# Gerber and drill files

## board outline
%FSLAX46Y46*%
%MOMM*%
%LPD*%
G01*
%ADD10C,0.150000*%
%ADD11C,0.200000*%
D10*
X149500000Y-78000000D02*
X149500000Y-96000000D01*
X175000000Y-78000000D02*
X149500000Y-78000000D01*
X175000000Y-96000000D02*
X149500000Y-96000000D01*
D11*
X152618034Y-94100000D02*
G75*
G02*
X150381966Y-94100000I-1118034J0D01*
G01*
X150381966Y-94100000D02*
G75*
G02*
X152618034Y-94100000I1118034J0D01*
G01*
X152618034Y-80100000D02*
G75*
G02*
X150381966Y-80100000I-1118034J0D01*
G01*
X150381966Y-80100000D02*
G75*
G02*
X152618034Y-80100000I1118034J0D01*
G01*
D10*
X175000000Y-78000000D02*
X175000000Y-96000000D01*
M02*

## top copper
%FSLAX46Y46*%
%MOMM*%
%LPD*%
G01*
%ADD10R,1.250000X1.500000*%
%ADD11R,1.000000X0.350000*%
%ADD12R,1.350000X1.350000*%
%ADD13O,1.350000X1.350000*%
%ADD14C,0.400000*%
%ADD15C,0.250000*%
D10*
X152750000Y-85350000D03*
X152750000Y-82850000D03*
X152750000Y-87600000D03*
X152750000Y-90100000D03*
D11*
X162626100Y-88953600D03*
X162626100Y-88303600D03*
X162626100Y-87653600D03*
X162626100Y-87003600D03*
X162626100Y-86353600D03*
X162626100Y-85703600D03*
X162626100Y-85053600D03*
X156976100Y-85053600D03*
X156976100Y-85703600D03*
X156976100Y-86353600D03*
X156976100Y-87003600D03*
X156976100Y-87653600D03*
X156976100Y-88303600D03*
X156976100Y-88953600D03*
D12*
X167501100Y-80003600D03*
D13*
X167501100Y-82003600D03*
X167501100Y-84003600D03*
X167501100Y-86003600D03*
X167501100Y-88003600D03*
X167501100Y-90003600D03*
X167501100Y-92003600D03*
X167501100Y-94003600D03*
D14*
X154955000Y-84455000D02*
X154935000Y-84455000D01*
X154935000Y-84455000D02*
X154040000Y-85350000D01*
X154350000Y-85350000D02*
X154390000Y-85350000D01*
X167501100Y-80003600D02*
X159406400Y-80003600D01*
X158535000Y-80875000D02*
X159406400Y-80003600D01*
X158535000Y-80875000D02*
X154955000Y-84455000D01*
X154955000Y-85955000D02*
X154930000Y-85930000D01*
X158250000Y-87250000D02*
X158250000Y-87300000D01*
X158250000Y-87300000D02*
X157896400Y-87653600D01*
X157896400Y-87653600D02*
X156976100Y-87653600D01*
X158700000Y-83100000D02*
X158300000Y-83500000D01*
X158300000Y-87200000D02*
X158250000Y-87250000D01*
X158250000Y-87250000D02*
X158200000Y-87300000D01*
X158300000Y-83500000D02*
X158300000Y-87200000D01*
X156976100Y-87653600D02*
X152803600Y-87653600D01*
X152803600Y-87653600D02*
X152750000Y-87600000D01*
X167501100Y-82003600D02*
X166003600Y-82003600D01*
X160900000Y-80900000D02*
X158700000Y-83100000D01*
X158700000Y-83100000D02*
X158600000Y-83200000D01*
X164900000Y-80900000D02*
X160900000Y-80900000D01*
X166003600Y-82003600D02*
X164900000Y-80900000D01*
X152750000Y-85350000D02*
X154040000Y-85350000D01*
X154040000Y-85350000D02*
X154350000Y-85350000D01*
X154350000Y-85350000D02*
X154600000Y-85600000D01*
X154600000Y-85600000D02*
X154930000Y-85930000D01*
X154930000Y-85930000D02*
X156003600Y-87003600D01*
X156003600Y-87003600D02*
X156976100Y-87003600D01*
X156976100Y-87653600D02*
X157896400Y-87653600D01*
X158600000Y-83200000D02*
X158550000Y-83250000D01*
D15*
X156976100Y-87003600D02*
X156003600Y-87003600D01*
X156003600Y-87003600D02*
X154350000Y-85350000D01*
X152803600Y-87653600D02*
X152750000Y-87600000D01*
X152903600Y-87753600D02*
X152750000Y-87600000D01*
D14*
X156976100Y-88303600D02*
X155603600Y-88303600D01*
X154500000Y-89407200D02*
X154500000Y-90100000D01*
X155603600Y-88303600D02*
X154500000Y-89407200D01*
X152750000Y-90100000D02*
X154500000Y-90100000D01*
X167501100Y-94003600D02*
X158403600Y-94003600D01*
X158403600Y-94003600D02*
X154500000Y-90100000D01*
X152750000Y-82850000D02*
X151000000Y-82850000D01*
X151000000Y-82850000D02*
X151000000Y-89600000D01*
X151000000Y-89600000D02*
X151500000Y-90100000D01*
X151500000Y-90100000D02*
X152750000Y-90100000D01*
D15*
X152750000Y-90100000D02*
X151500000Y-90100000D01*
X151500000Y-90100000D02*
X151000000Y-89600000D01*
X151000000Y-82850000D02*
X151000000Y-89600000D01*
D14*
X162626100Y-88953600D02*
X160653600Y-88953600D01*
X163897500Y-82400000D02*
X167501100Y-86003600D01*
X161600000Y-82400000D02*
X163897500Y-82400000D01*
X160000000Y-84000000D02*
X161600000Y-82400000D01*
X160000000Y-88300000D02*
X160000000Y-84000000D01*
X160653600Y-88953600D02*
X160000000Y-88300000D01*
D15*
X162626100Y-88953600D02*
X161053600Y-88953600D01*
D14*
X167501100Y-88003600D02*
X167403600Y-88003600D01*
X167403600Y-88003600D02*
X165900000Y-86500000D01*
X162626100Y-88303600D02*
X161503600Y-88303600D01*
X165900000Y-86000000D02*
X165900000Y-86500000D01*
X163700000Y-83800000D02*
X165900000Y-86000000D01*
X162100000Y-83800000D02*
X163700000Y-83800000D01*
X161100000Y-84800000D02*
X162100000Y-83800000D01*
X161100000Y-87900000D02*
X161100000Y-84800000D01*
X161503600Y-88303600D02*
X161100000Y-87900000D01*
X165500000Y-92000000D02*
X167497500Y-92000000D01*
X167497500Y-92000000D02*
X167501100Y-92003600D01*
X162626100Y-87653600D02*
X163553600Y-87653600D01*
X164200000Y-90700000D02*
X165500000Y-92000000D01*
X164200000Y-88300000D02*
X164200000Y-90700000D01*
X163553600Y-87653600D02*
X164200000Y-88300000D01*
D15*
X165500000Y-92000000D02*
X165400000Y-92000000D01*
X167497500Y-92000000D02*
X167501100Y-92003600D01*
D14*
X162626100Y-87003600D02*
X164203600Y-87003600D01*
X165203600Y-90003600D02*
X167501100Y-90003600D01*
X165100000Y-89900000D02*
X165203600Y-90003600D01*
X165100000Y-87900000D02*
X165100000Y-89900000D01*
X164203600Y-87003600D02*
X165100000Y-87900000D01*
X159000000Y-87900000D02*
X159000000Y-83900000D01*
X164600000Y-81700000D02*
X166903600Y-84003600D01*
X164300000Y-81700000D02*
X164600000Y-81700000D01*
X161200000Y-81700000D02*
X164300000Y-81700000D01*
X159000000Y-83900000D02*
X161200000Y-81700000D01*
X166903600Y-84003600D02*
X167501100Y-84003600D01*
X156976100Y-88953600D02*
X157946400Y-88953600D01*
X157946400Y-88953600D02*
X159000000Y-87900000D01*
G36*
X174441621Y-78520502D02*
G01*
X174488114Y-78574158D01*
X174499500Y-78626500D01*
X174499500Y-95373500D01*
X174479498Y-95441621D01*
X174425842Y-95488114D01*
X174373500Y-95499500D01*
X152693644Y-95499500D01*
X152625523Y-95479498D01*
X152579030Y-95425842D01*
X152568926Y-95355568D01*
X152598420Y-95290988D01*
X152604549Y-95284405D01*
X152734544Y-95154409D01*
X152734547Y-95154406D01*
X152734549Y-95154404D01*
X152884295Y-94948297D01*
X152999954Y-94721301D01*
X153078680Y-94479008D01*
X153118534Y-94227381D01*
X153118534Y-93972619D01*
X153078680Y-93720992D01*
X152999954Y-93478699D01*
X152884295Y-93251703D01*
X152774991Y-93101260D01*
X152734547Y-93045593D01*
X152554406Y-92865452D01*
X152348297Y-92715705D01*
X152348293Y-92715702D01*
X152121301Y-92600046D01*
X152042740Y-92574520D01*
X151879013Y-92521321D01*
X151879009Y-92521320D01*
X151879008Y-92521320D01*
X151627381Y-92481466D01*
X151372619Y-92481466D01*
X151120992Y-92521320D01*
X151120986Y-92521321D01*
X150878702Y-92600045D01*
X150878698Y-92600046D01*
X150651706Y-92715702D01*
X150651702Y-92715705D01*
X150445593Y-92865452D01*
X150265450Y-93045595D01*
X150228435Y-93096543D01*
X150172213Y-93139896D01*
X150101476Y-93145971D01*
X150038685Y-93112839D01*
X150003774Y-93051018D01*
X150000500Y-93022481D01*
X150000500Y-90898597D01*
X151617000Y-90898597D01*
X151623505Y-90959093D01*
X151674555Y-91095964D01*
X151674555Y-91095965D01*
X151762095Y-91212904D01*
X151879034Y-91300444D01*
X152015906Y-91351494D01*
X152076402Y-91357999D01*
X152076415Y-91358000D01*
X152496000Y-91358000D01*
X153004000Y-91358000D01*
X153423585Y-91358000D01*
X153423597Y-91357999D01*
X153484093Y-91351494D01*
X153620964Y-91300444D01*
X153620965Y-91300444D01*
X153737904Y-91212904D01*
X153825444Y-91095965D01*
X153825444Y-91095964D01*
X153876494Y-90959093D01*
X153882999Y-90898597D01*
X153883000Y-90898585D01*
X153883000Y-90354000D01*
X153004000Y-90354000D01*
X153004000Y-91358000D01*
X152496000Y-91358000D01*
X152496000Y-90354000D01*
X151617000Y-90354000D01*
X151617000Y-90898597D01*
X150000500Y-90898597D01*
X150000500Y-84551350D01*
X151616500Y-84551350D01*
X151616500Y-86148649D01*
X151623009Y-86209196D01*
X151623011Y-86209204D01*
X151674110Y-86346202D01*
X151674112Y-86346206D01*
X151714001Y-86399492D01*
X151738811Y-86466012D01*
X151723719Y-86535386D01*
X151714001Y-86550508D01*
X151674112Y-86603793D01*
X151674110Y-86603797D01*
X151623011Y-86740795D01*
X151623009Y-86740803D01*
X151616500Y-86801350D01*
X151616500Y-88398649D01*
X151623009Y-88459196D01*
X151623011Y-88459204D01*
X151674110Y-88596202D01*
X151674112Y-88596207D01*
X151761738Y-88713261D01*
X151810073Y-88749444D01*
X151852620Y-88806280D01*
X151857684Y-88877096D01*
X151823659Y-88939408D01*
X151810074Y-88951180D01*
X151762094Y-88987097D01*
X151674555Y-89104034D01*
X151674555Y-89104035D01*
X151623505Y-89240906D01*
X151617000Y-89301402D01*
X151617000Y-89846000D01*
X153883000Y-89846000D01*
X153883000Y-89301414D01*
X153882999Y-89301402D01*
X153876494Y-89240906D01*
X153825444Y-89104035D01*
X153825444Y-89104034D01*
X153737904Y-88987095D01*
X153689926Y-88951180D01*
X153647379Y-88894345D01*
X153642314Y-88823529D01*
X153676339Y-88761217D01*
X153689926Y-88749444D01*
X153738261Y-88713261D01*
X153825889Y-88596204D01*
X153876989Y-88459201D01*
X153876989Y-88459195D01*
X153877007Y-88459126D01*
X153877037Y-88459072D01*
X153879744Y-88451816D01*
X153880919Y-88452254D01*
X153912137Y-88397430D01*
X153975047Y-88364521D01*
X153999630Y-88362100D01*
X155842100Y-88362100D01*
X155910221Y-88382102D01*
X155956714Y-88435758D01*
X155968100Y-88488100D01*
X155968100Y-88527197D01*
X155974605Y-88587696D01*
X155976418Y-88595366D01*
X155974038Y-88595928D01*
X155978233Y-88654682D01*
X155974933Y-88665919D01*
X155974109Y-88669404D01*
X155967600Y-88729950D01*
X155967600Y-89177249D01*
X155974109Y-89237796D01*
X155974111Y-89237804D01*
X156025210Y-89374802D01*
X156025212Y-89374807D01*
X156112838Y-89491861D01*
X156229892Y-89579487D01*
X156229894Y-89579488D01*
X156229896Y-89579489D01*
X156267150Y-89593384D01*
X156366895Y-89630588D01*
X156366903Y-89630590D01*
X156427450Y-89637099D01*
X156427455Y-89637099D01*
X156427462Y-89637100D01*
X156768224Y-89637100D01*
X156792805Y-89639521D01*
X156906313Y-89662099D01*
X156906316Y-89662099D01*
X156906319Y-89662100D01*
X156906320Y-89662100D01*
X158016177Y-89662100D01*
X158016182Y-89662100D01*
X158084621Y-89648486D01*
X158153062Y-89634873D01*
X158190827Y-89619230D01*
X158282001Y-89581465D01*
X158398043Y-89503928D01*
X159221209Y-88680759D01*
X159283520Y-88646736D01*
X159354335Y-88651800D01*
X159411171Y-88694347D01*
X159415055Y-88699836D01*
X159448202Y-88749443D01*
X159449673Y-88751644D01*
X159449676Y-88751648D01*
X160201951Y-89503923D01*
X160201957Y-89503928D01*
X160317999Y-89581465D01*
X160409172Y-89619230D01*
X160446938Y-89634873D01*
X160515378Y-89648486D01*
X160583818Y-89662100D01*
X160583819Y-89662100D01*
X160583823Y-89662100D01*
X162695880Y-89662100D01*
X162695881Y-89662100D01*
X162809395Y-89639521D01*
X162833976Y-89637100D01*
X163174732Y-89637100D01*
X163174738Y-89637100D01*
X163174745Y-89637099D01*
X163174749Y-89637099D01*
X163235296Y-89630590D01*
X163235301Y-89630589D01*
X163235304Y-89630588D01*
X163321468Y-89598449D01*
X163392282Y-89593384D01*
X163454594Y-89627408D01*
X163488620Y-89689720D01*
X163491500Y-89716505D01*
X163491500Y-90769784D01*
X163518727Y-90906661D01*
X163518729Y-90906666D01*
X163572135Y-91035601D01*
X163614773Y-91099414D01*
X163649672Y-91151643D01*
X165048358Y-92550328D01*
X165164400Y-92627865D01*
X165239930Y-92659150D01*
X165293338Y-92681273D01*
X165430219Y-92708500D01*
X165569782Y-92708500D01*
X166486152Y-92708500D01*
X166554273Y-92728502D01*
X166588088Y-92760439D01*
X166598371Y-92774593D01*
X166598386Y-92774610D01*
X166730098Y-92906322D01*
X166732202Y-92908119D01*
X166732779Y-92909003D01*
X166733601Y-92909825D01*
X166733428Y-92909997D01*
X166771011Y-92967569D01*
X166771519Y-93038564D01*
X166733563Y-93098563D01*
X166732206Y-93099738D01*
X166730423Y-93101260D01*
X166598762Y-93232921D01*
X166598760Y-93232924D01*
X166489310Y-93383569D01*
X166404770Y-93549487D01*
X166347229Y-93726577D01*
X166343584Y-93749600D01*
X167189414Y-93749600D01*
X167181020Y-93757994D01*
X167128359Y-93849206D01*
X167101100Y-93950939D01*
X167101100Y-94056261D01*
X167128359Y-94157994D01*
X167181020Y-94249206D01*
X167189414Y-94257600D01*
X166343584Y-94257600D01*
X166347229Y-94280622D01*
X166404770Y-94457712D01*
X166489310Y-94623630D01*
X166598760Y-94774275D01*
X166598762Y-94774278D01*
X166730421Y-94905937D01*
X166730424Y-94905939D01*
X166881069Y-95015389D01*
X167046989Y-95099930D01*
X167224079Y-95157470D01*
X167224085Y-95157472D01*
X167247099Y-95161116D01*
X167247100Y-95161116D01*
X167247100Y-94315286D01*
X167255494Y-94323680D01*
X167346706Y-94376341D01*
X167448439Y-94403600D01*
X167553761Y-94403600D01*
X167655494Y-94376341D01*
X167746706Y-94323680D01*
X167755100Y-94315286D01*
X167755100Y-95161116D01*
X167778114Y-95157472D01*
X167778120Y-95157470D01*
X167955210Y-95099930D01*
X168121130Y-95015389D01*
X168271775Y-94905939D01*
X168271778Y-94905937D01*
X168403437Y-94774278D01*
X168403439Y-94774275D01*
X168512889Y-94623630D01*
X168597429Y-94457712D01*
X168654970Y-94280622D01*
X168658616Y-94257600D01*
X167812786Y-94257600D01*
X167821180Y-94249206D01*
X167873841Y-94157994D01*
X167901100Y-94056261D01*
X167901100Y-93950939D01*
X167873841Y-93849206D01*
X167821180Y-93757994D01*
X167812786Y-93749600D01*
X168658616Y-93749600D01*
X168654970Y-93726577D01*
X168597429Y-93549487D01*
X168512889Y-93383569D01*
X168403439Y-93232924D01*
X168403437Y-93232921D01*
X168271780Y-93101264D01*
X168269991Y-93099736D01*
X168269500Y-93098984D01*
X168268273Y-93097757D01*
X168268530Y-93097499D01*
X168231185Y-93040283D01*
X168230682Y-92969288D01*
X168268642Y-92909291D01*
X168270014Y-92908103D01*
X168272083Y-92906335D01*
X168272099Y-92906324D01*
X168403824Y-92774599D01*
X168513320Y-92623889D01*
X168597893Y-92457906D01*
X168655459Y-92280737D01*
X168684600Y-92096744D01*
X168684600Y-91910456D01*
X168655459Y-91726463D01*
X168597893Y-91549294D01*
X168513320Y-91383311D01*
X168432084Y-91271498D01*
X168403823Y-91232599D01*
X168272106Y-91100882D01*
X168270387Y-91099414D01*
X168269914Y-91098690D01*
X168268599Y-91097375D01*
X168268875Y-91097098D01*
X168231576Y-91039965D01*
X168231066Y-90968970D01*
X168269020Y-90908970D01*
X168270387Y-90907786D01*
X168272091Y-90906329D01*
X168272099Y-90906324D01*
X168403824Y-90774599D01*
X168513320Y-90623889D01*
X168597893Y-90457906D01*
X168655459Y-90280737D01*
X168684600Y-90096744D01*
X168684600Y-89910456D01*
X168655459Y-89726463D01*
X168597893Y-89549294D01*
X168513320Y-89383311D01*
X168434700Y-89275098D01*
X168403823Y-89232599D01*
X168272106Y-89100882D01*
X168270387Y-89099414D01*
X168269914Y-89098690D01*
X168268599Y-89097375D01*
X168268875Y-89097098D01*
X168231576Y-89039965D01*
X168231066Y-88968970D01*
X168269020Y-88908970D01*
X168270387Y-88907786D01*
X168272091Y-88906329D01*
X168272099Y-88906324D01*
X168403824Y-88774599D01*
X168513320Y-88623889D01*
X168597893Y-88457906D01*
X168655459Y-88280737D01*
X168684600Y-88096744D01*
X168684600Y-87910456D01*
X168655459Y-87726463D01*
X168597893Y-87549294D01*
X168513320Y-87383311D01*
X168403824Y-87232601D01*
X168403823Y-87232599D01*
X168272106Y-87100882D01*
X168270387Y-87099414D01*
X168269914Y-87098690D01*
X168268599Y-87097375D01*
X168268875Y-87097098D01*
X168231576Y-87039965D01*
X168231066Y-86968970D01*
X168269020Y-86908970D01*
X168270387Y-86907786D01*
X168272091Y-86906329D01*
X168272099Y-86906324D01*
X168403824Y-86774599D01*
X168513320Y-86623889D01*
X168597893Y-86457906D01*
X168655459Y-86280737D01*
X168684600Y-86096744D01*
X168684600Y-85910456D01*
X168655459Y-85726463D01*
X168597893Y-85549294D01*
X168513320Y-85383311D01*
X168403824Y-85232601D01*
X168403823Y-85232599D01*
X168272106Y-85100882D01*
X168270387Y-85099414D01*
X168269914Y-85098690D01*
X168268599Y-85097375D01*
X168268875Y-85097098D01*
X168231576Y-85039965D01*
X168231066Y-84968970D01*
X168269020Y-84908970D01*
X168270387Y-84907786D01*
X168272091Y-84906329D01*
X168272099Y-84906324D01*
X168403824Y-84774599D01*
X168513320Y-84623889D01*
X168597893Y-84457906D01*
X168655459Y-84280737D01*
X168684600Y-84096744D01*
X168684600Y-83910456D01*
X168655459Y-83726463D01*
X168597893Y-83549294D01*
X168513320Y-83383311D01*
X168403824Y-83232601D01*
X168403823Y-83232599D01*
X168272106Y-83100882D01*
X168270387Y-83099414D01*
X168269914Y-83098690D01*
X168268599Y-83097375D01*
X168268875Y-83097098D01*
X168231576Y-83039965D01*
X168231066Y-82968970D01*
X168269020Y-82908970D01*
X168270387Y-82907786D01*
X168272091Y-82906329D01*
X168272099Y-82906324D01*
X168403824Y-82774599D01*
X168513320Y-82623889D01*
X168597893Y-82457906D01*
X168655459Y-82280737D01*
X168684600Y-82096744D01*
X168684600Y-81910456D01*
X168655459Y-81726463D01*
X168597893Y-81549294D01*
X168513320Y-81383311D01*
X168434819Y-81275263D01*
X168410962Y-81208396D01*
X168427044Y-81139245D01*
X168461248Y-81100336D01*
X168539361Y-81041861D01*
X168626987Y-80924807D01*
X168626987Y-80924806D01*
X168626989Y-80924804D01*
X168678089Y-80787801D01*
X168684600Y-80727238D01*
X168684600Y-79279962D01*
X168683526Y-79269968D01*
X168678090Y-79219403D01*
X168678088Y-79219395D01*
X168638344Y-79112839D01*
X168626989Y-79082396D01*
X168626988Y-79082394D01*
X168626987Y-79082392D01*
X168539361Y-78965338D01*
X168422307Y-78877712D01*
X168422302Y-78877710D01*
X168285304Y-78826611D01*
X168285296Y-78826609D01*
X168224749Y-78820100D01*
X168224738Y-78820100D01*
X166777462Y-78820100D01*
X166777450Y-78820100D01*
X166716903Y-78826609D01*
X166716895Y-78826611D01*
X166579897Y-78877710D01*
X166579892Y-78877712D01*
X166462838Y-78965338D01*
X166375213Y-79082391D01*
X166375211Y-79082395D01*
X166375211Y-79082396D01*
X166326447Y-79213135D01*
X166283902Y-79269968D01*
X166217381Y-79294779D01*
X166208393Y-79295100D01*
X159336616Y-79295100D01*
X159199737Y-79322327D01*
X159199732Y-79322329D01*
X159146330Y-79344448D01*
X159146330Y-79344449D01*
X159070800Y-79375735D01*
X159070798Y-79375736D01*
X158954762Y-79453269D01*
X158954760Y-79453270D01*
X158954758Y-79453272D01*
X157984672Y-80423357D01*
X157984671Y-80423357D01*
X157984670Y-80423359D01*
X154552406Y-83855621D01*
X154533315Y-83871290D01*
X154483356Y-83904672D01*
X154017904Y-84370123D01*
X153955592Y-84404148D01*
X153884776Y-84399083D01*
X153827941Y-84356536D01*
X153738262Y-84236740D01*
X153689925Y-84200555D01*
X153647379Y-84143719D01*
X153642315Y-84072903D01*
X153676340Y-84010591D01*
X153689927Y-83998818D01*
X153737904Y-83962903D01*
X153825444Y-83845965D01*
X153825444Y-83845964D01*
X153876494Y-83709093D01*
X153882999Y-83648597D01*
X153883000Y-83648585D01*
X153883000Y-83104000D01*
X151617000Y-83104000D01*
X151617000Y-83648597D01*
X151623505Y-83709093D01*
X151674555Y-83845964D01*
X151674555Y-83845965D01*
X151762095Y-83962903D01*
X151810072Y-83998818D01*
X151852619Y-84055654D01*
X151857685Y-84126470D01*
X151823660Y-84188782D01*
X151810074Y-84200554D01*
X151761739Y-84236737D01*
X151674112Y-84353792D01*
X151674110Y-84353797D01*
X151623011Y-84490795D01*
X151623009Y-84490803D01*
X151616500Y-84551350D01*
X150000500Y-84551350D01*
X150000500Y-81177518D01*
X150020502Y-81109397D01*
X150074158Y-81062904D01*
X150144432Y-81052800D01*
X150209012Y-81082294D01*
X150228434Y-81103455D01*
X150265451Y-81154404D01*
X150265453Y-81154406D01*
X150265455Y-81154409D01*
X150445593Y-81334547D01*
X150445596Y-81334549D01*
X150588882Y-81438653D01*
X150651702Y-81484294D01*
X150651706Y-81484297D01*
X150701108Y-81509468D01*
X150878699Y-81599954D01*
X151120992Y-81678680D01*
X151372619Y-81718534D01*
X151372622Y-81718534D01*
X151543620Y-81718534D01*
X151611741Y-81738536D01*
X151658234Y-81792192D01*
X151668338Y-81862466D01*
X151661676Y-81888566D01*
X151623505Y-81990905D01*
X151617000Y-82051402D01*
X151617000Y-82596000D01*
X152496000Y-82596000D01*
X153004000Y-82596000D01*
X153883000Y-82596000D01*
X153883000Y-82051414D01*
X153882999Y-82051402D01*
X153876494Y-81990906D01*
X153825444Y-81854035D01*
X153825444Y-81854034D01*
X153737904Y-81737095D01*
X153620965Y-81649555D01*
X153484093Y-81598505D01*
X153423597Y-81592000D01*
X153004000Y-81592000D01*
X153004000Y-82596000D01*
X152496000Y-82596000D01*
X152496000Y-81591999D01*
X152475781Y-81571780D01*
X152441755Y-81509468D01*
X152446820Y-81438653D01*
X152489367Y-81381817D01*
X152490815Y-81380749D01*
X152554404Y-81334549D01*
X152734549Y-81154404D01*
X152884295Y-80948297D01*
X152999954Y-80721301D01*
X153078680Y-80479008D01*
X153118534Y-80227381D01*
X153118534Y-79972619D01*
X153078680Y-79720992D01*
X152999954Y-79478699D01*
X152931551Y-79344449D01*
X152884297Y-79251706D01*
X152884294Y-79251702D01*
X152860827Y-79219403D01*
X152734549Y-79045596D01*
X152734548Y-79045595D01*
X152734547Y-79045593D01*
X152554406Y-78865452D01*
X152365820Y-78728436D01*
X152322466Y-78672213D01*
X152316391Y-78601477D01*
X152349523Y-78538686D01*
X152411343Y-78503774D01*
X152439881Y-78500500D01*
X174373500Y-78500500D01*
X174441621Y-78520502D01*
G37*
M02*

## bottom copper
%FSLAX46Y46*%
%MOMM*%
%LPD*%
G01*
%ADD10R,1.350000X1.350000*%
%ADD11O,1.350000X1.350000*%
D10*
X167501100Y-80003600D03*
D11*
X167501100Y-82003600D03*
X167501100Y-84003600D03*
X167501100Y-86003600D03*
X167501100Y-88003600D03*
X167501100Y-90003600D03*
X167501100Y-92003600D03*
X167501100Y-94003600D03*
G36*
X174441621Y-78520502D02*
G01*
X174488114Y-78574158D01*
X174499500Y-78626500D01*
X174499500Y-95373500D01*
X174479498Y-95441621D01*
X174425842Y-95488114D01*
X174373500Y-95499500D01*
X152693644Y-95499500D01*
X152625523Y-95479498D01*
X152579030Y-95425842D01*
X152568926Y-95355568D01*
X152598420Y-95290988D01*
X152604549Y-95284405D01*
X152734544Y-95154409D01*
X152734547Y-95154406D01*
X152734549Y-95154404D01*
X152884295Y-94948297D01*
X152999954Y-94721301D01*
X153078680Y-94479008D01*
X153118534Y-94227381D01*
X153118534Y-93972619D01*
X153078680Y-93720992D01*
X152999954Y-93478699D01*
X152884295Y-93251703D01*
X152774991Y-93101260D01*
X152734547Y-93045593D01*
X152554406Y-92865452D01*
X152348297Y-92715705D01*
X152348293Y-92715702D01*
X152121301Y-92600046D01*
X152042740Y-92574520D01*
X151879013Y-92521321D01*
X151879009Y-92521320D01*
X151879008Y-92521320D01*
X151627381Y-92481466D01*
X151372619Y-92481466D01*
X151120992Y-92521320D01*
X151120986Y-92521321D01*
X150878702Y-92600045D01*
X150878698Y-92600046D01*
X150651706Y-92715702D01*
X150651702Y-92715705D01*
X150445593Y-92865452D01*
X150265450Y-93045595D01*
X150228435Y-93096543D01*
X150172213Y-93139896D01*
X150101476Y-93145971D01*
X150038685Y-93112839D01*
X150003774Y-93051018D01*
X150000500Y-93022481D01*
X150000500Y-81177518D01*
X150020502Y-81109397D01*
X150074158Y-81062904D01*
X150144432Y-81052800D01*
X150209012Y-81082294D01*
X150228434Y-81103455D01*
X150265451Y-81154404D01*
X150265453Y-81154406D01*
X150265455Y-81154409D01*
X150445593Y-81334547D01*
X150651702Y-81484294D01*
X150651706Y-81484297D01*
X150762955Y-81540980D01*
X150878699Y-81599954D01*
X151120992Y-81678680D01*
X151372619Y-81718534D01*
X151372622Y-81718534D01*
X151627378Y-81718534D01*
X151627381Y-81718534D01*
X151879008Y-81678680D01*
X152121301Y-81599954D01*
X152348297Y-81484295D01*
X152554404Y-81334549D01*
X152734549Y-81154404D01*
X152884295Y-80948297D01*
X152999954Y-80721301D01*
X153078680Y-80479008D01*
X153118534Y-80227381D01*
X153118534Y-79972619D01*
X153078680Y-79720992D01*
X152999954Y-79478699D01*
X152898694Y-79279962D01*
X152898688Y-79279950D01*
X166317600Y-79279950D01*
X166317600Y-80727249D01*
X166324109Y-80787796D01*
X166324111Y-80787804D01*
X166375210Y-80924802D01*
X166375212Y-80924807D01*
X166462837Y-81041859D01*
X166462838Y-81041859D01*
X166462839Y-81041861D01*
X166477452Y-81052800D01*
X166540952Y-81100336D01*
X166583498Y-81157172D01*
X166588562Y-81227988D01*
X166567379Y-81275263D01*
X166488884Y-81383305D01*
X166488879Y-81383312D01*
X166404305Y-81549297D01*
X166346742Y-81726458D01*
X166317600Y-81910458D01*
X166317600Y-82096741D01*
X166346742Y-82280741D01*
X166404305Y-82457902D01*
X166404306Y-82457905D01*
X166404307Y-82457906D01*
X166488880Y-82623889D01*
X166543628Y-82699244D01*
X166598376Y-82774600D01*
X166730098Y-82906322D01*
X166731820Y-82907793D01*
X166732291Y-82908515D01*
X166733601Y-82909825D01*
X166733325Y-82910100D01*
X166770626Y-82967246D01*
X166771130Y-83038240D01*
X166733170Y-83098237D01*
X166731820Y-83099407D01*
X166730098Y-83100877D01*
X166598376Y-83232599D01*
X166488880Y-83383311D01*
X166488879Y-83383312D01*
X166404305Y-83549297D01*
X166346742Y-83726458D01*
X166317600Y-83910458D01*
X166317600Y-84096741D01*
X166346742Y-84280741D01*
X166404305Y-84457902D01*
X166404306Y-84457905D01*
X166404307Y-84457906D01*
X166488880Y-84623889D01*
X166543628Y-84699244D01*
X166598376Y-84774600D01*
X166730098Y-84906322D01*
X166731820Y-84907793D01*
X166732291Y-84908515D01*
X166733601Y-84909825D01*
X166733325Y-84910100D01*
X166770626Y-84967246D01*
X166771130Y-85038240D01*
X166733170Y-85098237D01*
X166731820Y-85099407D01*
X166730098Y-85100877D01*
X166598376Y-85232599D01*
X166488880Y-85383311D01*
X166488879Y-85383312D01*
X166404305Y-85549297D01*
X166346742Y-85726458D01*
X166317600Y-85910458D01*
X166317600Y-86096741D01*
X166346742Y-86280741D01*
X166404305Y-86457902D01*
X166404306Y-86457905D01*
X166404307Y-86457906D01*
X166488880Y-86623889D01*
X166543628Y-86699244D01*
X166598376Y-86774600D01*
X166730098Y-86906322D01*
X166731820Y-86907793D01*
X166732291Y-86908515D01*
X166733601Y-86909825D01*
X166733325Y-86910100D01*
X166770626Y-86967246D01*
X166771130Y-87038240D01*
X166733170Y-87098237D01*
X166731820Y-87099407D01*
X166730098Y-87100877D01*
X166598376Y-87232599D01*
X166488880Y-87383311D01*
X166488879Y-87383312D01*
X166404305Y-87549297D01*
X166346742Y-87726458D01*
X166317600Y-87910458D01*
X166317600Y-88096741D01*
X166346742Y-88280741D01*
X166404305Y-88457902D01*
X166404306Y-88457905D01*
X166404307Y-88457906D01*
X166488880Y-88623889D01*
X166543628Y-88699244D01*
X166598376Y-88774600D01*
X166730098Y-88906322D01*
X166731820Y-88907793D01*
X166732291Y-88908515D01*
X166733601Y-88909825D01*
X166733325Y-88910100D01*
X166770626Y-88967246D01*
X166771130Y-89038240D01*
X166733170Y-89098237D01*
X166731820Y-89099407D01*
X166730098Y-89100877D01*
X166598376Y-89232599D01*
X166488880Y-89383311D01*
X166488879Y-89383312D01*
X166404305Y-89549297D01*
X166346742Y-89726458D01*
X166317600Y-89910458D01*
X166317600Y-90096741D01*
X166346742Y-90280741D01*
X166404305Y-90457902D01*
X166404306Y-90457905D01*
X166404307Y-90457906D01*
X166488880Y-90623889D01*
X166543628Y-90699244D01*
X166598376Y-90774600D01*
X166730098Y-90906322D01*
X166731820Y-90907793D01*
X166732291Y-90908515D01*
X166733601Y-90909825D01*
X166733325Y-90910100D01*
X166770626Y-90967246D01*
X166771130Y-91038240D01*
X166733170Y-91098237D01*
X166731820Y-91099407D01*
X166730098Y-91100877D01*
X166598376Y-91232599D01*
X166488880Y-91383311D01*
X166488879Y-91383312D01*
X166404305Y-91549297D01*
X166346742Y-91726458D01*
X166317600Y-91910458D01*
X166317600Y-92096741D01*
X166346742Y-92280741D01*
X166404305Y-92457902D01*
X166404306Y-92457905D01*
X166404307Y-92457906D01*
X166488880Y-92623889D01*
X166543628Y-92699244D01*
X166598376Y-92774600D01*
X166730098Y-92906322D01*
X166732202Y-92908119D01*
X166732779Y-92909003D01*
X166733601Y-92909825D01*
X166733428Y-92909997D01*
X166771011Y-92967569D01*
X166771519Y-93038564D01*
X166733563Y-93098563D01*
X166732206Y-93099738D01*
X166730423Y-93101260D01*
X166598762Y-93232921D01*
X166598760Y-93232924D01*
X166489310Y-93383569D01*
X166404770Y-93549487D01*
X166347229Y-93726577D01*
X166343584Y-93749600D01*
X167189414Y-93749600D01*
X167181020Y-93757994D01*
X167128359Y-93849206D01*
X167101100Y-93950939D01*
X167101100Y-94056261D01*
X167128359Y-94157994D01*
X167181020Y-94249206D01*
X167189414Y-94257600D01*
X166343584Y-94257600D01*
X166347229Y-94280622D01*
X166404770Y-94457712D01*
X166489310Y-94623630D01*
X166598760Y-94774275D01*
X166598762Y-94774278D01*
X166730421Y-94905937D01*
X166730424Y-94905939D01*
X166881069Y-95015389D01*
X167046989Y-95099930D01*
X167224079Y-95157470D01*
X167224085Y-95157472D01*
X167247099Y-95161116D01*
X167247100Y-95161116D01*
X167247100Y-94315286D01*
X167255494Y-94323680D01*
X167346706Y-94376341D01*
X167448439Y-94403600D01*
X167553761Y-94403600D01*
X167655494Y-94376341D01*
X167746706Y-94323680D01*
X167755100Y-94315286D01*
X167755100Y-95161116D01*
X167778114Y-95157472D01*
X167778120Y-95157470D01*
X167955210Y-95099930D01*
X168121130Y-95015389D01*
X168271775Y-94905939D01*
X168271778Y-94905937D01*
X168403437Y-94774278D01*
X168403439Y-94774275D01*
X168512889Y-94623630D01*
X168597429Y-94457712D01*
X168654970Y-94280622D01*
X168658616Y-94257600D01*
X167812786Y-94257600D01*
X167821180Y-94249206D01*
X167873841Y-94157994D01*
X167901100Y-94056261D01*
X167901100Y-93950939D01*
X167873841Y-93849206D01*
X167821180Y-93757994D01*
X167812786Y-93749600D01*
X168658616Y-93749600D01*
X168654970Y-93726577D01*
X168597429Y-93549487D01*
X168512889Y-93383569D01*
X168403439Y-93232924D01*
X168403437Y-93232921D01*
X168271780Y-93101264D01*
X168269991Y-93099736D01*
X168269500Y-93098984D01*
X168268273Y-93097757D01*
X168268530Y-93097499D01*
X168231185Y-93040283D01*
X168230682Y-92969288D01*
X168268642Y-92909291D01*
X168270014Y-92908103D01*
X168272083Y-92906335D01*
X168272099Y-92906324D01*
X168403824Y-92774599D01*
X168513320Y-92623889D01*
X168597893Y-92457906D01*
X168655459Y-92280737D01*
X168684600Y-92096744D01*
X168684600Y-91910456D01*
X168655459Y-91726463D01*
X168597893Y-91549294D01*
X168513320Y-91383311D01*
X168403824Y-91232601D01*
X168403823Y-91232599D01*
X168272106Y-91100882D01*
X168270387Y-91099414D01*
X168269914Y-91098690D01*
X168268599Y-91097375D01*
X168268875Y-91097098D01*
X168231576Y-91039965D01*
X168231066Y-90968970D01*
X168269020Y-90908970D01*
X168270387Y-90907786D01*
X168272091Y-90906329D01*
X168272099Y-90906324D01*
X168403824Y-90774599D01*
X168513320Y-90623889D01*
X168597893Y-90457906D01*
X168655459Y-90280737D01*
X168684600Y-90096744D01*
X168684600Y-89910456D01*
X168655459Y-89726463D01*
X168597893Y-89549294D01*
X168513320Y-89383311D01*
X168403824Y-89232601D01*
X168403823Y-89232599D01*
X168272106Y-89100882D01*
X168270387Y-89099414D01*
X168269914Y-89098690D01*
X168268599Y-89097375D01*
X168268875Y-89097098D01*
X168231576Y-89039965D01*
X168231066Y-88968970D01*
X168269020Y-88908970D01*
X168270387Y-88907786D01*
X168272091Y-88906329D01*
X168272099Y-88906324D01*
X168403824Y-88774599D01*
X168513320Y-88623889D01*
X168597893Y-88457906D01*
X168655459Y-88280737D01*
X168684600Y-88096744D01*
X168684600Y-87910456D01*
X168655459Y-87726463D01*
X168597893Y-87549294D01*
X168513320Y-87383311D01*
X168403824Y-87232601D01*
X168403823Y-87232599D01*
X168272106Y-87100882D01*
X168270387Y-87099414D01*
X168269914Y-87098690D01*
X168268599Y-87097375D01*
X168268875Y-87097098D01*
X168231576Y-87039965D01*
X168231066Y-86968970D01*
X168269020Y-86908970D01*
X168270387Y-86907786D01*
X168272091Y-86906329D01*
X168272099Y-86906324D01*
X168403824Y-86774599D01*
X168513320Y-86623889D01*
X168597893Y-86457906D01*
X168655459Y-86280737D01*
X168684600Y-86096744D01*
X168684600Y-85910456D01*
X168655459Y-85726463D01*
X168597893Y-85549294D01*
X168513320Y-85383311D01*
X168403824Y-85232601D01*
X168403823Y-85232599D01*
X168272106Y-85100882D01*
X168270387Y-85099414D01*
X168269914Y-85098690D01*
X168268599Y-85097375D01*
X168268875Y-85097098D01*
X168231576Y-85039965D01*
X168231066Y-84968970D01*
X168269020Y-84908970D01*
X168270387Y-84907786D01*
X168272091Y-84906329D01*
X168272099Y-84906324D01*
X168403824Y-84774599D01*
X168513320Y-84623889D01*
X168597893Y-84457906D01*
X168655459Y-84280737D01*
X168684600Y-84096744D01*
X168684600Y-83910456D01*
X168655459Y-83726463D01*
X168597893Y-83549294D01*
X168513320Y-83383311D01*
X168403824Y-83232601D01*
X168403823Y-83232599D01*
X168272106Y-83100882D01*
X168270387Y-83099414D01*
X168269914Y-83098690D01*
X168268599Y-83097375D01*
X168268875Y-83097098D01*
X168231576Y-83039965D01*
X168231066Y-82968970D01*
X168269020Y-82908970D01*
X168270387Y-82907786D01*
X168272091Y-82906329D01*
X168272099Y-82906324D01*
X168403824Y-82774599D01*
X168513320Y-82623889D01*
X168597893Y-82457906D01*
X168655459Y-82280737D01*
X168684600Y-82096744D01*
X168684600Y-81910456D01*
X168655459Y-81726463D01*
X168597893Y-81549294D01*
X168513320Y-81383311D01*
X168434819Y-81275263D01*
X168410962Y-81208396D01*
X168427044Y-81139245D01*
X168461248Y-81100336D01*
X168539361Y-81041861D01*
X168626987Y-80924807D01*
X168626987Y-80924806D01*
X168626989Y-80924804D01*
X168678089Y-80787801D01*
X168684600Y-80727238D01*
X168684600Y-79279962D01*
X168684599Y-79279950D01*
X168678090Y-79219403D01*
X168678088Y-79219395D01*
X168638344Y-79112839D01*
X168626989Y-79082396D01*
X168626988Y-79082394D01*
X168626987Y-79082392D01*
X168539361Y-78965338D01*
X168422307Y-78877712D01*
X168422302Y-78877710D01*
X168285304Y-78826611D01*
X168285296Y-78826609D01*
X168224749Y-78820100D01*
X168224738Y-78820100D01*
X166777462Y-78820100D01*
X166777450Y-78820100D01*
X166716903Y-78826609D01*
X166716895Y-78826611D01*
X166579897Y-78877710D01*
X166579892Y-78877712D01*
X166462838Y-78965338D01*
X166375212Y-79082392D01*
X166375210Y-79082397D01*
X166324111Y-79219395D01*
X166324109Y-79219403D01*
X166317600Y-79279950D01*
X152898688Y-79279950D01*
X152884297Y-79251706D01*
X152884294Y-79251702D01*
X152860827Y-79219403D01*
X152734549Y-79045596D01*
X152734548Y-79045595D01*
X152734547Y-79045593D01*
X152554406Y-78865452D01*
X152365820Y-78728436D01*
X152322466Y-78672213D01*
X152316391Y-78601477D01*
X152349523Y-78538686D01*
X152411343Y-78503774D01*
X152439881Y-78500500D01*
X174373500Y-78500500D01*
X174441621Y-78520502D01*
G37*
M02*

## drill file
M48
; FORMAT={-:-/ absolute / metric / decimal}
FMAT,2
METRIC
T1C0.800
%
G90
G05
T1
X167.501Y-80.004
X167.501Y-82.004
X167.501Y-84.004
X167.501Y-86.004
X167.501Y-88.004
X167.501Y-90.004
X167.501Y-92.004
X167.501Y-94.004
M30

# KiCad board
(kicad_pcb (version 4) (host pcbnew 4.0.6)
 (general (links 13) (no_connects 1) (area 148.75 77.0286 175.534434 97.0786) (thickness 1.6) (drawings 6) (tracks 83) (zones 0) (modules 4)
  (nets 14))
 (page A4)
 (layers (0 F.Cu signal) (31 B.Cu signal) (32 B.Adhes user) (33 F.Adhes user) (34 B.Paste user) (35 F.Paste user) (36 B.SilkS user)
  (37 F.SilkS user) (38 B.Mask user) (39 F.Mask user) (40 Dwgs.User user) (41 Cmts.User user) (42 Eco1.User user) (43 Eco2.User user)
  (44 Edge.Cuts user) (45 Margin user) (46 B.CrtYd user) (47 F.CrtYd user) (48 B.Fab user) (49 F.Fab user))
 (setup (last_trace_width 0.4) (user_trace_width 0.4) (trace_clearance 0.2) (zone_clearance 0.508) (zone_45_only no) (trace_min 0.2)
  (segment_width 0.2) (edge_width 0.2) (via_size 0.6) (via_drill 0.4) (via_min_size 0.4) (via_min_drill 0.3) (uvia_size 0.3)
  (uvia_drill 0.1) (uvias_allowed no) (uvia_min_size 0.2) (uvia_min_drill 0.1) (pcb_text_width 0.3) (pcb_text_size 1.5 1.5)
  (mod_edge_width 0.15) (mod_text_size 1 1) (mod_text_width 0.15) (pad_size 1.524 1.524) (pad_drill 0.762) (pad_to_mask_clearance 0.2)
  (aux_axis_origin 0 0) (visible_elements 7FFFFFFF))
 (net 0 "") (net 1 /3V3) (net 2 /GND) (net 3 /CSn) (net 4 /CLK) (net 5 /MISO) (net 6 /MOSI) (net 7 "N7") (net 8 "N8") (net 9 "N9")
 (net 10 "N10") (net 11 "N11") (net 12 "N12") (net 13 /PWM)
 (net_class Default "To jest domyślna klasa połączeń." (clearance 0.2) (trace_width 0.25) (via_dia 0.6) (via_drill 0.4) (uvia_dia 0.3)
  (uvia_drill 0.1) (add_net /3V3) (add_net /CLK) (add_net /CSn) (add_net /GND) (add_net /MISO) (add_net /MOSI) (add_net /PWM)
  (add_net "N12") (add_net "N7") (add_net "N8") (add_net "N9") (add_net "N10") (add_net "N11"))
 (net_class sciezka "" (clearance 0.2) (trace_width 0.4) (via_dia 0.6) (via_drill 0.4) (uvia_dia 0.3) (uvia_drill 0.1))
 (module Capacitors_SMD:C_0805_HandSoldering (layer F.Cu) (at 152.75 84.1 90)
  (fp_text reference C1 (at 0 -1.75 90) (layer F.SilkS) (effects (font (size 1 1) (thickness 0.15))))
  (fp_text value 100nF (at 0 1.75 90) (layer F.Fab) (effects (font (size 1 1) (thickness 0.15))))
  (pad 1 smd rect (at -1.25 0 90) (size 1.5 1.25) (layers F.Cu F.Paste F.Mask) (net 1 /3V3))
  (pad 2 smd rect (at 1.25 0 90) (size 1.5 1.25) (layers F.Cu F.Paste F.Mask) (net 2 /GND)))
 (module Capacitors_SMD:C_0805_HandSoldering (layer F.Cu) (at 152.75 88.85 270)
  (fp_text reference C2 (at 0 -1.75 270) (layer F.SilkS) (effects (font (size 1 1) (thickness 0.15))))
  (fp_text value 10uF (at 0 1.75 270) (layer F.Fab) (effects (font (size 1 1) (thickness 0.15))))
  (pad 1 smd rect (at -1.25 0 270) (size 1.5 1.25) (layers F.Cu F.Paste F.Mask) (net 1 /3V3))
  (pad 2 smd rect (at 1.25 0 270) (size 1.5 1.25) (layers F.Cu F.Paste F.Mask) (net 2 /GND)))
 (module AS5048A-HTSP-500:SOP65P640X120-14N (layer F.Cu) (at 159.8011 87.0036 180) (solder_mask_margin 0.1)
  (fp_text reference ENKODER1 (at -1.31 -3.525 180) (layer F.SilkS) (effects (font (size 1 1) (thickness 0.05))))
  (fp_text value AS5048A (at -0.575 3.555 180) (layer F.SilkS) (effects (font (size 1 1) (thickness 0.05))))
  (pad 1 smd rect (at -2.825 -1.95 90) (size 0.35 1) (layers F.Cu F.Paste F.Mask) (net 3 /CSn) (solder_mask_margin 0.2))
  (pad 2 smd rect (at -2.825 -1.3 90) (size 0.35 1) (layers F.Cu F.Paste F.Mask) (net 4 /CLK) (solder_mask_margin 0.2))
  (pad 3 smd rect (at -2.825 -0.65 90) (size 0.35 1) (layers F.Cu F.Paste F.Mask) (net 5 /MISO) (solder_mask_margin 0.2))
  (pad 4 smd rect (at -2.825 0 90) (size 0.35 1) (layers F.Cu F.Paste F.Mask) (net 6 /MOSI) (solder_mask_margin 0.2))
  (pad 5 smd rect (at -2.825 0.65 90) (size 0.35 1) (layers F.Cu F.Paste F.Mask) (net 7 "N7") (solder_mask_margin 0.2))
  (pad 6 smd rect (at -2.825 1.3 90) (size 0.35 1) (layers F.Cu F.Paste F.Mask) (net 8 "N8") (solder_mask_margin 0.2))
  (pad 7 smd rect (at -2.825 1.95 90) (size 0.35 1) (layers F.Cu F.Paste F.Mask) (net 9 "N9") (solder_mask_margin 0.2))
  (pad 8 smd rect (at 2.825 1.95 270) (size 0.35 1) (layers F.Cu F.Paste F.Mask) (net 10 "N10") (solder_mask_margin 0.2))
  (pad 9 smd rect (at 2.825 1.3 270) (size 0.35 1) (layers F.Cu F.Paste F.Mask) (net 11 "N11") (solder_mask_margin 0.2))
  (pad 10 smd rect (at 2.825 0.65 270) (size 0.35 1) (layers F.Cu F.Paste F.Mask) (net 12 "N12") (solder_mask_margin 0.2))
  (pad 11 smd rect (at 2.825 0 270) (size 0.35 1) (layers F.Cu F.Paste F.Mask) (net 1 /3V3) (solder_mask_margin 0.2))
  (pad 12 smd rect (at 2.825 -0.65 270) (size 0.35 1) (layers F.Cu F.Paste F.Mask) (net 1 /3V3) (solder_mask_margin 0.2))
  (pad 13 smd rect (at 2.825 -1.3 270) (size 0.35 1) (layers F.Cu F.Paste F.Mask) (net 2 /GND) (solder_mask_margin 0.2))
  (pad 14 smd rect (at 2.825 -1.95 270) (size 0.35 1) (layers F.Cu F.Paste F.Mask) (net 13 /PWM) (solder_mask_margin 0.2)))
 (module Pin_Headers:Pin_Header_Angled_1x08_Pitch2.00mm (layer F.Cu) (at 167.5011 80.0036)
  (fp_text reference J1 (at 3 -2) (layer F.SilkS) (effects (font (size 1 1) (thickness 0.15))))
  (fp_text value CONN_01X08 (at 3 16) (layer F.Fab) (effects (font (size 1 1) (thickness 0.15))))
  (pad 1 thru_hole rect (at 0 0) (size 1.35 1.35) (drill 0.8) (layers *.Cu *.Mask) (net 1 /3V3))
  (pad 2 thru_hole oval (at 0 2) (size 1.35 1.35) (drill 0.8) (layers *.Cu *.Mask) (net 1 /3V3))
  (pad 3 thru_hole oval (at 0 4) (size 1.35 1.35) (drill 0.8) (layers *.Cu *.Mask) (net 13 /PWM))
  (pad 4 thru_hole oval (at 0 6) (size 1.35 1.35) (drill 0.8) (layers *.Cu *.Mask) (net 3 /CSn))
  (pad 5 thru_hole oval (at 0 8) (size 1.35 1.35) (drill 0.8) (layers *.Cu *.Mask) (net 4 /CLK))
  (pad 6 thru_hole oval (at 0 10) (size 1.35 1.35) (drill 0.8) (layers *.Cu *.Mask) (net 6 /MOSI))
  (pad 7 thru_hole oval (at 0 12) (size 1.35 1.35) (drill 0.8) (layers *.Cu *.Mask) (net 5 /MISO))
  (pad 8 thru_hole oval (at 0 14) (size 1.35 1.35) (drill 0.8) (layers *.Cu *.Mask) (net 2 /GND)))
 (gr_line (start 149.5 78) (end 149.5 96) (angle 90) (layer Edge.Cuts) (width 0.15))
 (gr_line (start 175 78) (end 149.5 78) (angle 90) (layer Edge.Cuts) (width 0.15))
 (gr_line (start 175 96) (end 149.5 96) (angle 90) (layer Edge.Cuts) (width 0.15))
 (gr_circle (center 151.5 94.1) (end 152.5 94.6) (layer Edge.Cuts) (width 0.2))
 (gr_circle (center 151.5 80.1) (end 152 81.1) (layer Edge.Cuts) (width 0.2))
 (gr_line (start 175 78) (end 175 96) (angle 90) (layer Edge.Cuts) (width 0.15))
 (segment (start 154.955 84.455) (end 154.935 84.455) (width 0.4) (layer F.Cu) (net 1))
 (segment (start 154.935 84.455) (end 154.04 85.35) (width 0.4) (layer F.Cu) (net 1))
 (segment (start 154.35 85.35) (end 154.39 85.35) (width 0.4) (layer F.Cu) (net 1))
 (segment (start 167.5011 80.0036) (end 159.4064 80.0036) (width 0.4) (layer F.Cu) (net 1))
 (segment (start 158.535 80.875) (end 159.4064 80.0036) (width 0.4) (layer F.Cu) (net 1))
 (segment (start 158.535 80.875) (end 154.955 84.455) (width 0.4) (layer F.Cu) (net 1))
 (segment (start 154.955 85.955) (end 154.93 85.93) (width 0.4) (layer F.Cu) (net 1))
 (segment (start 158.25 87.25) (end 158.25 87.3) (width 0.4) (layer F.Cu) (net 1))
 (segment (start 158.25 87.3) (end 157.8964 87.6536) (width 0.4) (layer F.Cu) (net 1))
 (segment (start 157.8964 87.6536) (end 156.9761 87.6536) (width 0.4) (layer F.Cu) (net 1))
 (segment (start 158.7 83.1) (end 158.3 83.5) (width 0.4) (layer F.Cu) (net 1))
 (segment (start 158.3 87.2) (end 158.25 87.25) (width 0.4) (layer F.Cu) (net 1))
 (segment (start 158.25 87.25) (end 158.2 87.3) (width 0.4) (layer F.Cu) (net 1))
 (segment (start 158.3 83.5) (end 158.3 87.2) (width 0.4) (layer F.Cu) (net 1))
 (segment (start 156.9761 87.6536) (end 152.8036 87.6536) (width 0.4) (layer F.Cu) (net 1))
 (segment (start 152.8036 87.6536) (end 152.75 87.6) (width 0.4) (layer F.Cu) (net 1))
 (segment (start 167.5011 82.0036) (end 166.0036 82.0036) (width 0.4) (layer F.Cu) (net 1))
 (segment (start 160.9 80.9) (end 158.7 83.1) (width 0.4) (layer F.Cu) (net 1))
 (segment (start 158.7 83.1) (end 158.6 83.2) (width 0.4) (layer F.Cu) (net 1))
 (segment (start 164.9 80.9) (end 160.9 80.9) (width 0.4) (layer F.Cu) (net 1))
 (segment (start 166.0036 82.0036) (end 164.9 80.9) (width 0.4) (layer F.Cu) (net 1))
 (segment (start 152.75 85.35) (end 154.04 85.35) (width 0.4) (layer F.Cu) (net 1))
 (segment (start 154.04 85.35) (end 154.35 85.35) (width 0.4) (layer F.Cu) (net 1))
 (segment (start 154.35 85.35) (end 154.6 85.6) (width 0.4) (layer F.Cu) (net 1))
 (segment (start 154.6 85.6) (end 154.93 85.93) (width 0.4) (layer F.Cu) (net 1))
 (segment (start 154.93 85.93) (end 156.0036 87.0036) (width 0.4) (layer F.Cu) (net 1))
 (segment (start 156.0036 87.0036) (end 156.9761 87.0036) (width 0.4) (layer F.Cu) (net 1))
 (segment (start 156.9761 87.6536) (end 157.8964 87.6536) (width 0.4) (layer F.Cu) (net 1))
 (segment (start 158.6 83.2) (end 158.55 83.25) (width 0.4) (layer F.Cu) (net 1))
 (segment (start 156.9761 87.0036) (end 156.0036 87.0036) (width 0.25) (layer F.Cu) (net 1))
 (segment (start 156.0036 87.0036) (end 154.35 85.35) (width 0.25) (layer F.Cu) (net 1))
 (segment (start 152.8036 87.6536) (end 152.75 87.6) (width 0.25) (layer F.Cu) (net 1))
 (segment (start 152.9036 87.7536) (end 152.75 87.6) (width 0.25) (layer F.Cu) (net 1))
 (segment (start 156.9761 88.3036) (end 155.6036 88.3036) (width 0.4) (layer F.Cu) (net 2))
 (segment (start 154.5 89.4072) (end 154.5 90.1) (width 0.4) (layer F.Cu) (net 2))
 (segment (start 155.6036 88.3036) (end 154.5 89.4072) (width 0.4) (layer F.Cu) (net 2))
 (segment (start 152.75 90.1) (end 154.5 90.1) (width 0.4) (layer F.Cu) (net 2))
 (segment (start 167.5011 94.0036) (end 158.4036 94.0036) (width 0.4) (layer F.Cu) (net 2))
 (segment (start 158.4036 94.0036) (end 154.5 90.1) (width 0.4) (layer F.Cu) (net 2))
 (segment (start 152.75 82.85) (end 151 82.85) (width 0.4) (layer F.Cu) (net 2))
 (segment (start 151 82.85) (end 151 89.6) (width 0.4) (layer F.Cu) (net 2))
 (segment (start 151 89.6) (end 151.5 90.1) (width 0.4) (layer F.Cu) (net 2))
 (segment (start 151.5 90.1) (end 152.75 90.1) (width 0.4) (layer F.Cu) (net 2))
 (segment (start 152.75 90.1) (end 151.5 90.1) (width 0.25) (layer F.Cu) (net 2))
 (segment (start 151.5 90.1) (end 151 89.6) (width 0.25) (layer F.Cu) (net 2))
 (segment (start 151 82.85) (end 151 89.6) (width 0.25) (layer F.Cu) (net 2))
 (segment (start 162.6261 88.9536) (end 160.6536 88.9536) (width 0.4) (layer F.Cu) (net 3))
 (segment (start 163.8975 82.4) (end 167.5011 86.0036) (width 0.4) (layer F.Cu) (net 3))
 (segment (start 161.6 82.4) (end 163.8975 82.4) (width 0.4) (layer F.Cu) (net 3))
 (segment (start 160 84) (end 161.6 82.4) (width 0.4) (layer F.Cu) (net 3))
 (segment (start 160 88.3) (end 160 84) (width 0.4) (layer F.Cu) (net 3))
 (segment (start 160.6536 88.9536) (end 160 88.3) (width 0.4) (layer F.Cu) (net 3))
 (segment (start 162.6261 88.9536) (end 161.0536 88.9536) (width 0.25) (layer F.Cu) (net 3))
 (segment (start 167.5011 88.0036) (end 167.4036 88.0036) (width 0.4) (layer F.Cu) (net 4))
 (segment (start 167.4036 88.0036) (end 165.9 86.5) (width 0.4) (layer F.Cu) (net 4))
 (segment (start 162.6261 88.3036) (end 161.5036 88.3036) (width 0.4) (layer F.Cu) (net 4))
 (segment (start 165.9 86) (end 165.9 86.5) (width 0.4) (layer F.Cu) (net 4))
 (segment (start 163.7 83.8) (end 165.9 86) (width 0.4) (layer F.Cu) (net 4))
 (segment (start 162.1 83.8) (end 163.7 83.8) (width 0.4) (layer F.Cu) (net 4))
 (segment (start 161.1 84.8) (end 162.1 83.8) (width 0.4) (layer F.Cu) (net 4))
 (segment (start 161.1 87.9) (end 161.1 84.8) (width 0.4) (layer F.Cu) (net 4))
 (segment (start 161.5036 88.3036) (end 161.1 87.9) (width 0.4) (layer F.Cu) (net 4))
 (segment (start 165.5 92) (end 167.4975 92) (width 0.4) (layer F.Cu) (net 5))
 (segment (start 167.4975 92) (end 167.5011 92.0036) (width 0.4) (layer F.Cu) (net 5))
 (segment (start 162.6261 87.6536) (end 163.5536 87.6536) (width 0.4) (layer F.Cu) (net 5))
 (segment (start 164.2 90.7) (end 165.5 92) (width 0.4) (layer F.Cu) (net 5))
 (segment (start 164.2 88.3) (end 164.2 90.7) (width 0.4) (layer F.Cu) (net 5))
 (segment (start 163.5536 87.6536) (end 164.2 88.3) (width 0.4) (layer F.Cu) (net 5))
 (segment (start 165.5 92) (end 165.4 92) (width 0.25) (layer F.Cu) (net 5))
 (segment (start 167.4975 92) (end 167.5011 92.0036) (width 0.25) (layer F.Cu) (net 5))
 (segment (start 162.6261 87.0036) (end 164.2036 87.0036) (width 0.4) (layer F.Cu) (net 6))
 (segment (start 165.2036 90.0036) (end 167.5011 90.0036) (width 0.4) (layer F.Cu) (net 6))
 (segment (start 165.1 89.9) (end 165.2036 90.0036) (width 0.4) (layer F.Cu) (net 6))
 (segment (start 165.1 87.9) (end 165.1 89.9) (width 0.4) (layer F.Cu) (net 6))
 (segment (start 164.2036 87.0036) (end 165.1 87.9) (width 0.4) (layer F.Cu) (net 6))
 (segment (start 159 87.9) (end 159 83.9) (width 0.4) (layer F.Cu) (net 13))
 (segment (start 164.6 81.7) (end 166.9036 84.0036) (width 0.4) (layer F.Cu) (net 13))
 (segment (start 164.3 81.7) (end 164.6 81.7) (width 0.4) (layer F.Cu) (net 13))
 (segment (start 161.2 81.7) (end 164.3 81.7) (width 0.4) (layer F.Cu) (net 13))
 (segment (start 159 83.9) (end 161.2 81.7) (width 0.4) (layer F.Cu) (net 13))
 (segment (start 166.9036 84.0036) (end 167.5011 84.0036) (width 0.4) (layer F.Cu) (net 13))
 (segment (start 156.9761 88.9536) (end 157.9464 88.9536) (width 0.4) (layer F.Cu) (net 13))
 (segment (start 157.9464 88.9536) (end 159 87.9) (width 0.4) (layer F.Cu) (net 13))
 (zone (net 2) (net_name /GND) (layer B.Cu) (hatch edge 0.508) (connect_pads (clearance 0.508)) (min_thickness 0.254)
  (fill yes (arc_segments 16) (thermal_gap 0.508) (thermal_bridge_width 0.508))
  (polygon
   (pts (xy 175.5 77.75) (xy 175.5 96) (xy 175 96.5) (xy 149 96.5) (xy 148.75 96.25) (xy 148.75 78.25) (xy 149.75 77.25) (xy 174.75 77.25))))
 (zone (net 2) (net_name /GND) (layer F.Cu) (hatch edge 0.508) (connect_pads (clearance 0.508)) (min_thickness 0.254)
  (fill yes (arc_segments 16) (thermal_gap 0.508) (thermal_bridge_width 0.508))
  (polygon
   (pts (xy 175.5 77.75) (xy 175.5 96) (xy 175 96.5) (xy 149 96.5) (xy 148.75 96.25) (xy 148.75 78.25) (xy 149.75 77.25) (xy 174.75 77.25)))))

